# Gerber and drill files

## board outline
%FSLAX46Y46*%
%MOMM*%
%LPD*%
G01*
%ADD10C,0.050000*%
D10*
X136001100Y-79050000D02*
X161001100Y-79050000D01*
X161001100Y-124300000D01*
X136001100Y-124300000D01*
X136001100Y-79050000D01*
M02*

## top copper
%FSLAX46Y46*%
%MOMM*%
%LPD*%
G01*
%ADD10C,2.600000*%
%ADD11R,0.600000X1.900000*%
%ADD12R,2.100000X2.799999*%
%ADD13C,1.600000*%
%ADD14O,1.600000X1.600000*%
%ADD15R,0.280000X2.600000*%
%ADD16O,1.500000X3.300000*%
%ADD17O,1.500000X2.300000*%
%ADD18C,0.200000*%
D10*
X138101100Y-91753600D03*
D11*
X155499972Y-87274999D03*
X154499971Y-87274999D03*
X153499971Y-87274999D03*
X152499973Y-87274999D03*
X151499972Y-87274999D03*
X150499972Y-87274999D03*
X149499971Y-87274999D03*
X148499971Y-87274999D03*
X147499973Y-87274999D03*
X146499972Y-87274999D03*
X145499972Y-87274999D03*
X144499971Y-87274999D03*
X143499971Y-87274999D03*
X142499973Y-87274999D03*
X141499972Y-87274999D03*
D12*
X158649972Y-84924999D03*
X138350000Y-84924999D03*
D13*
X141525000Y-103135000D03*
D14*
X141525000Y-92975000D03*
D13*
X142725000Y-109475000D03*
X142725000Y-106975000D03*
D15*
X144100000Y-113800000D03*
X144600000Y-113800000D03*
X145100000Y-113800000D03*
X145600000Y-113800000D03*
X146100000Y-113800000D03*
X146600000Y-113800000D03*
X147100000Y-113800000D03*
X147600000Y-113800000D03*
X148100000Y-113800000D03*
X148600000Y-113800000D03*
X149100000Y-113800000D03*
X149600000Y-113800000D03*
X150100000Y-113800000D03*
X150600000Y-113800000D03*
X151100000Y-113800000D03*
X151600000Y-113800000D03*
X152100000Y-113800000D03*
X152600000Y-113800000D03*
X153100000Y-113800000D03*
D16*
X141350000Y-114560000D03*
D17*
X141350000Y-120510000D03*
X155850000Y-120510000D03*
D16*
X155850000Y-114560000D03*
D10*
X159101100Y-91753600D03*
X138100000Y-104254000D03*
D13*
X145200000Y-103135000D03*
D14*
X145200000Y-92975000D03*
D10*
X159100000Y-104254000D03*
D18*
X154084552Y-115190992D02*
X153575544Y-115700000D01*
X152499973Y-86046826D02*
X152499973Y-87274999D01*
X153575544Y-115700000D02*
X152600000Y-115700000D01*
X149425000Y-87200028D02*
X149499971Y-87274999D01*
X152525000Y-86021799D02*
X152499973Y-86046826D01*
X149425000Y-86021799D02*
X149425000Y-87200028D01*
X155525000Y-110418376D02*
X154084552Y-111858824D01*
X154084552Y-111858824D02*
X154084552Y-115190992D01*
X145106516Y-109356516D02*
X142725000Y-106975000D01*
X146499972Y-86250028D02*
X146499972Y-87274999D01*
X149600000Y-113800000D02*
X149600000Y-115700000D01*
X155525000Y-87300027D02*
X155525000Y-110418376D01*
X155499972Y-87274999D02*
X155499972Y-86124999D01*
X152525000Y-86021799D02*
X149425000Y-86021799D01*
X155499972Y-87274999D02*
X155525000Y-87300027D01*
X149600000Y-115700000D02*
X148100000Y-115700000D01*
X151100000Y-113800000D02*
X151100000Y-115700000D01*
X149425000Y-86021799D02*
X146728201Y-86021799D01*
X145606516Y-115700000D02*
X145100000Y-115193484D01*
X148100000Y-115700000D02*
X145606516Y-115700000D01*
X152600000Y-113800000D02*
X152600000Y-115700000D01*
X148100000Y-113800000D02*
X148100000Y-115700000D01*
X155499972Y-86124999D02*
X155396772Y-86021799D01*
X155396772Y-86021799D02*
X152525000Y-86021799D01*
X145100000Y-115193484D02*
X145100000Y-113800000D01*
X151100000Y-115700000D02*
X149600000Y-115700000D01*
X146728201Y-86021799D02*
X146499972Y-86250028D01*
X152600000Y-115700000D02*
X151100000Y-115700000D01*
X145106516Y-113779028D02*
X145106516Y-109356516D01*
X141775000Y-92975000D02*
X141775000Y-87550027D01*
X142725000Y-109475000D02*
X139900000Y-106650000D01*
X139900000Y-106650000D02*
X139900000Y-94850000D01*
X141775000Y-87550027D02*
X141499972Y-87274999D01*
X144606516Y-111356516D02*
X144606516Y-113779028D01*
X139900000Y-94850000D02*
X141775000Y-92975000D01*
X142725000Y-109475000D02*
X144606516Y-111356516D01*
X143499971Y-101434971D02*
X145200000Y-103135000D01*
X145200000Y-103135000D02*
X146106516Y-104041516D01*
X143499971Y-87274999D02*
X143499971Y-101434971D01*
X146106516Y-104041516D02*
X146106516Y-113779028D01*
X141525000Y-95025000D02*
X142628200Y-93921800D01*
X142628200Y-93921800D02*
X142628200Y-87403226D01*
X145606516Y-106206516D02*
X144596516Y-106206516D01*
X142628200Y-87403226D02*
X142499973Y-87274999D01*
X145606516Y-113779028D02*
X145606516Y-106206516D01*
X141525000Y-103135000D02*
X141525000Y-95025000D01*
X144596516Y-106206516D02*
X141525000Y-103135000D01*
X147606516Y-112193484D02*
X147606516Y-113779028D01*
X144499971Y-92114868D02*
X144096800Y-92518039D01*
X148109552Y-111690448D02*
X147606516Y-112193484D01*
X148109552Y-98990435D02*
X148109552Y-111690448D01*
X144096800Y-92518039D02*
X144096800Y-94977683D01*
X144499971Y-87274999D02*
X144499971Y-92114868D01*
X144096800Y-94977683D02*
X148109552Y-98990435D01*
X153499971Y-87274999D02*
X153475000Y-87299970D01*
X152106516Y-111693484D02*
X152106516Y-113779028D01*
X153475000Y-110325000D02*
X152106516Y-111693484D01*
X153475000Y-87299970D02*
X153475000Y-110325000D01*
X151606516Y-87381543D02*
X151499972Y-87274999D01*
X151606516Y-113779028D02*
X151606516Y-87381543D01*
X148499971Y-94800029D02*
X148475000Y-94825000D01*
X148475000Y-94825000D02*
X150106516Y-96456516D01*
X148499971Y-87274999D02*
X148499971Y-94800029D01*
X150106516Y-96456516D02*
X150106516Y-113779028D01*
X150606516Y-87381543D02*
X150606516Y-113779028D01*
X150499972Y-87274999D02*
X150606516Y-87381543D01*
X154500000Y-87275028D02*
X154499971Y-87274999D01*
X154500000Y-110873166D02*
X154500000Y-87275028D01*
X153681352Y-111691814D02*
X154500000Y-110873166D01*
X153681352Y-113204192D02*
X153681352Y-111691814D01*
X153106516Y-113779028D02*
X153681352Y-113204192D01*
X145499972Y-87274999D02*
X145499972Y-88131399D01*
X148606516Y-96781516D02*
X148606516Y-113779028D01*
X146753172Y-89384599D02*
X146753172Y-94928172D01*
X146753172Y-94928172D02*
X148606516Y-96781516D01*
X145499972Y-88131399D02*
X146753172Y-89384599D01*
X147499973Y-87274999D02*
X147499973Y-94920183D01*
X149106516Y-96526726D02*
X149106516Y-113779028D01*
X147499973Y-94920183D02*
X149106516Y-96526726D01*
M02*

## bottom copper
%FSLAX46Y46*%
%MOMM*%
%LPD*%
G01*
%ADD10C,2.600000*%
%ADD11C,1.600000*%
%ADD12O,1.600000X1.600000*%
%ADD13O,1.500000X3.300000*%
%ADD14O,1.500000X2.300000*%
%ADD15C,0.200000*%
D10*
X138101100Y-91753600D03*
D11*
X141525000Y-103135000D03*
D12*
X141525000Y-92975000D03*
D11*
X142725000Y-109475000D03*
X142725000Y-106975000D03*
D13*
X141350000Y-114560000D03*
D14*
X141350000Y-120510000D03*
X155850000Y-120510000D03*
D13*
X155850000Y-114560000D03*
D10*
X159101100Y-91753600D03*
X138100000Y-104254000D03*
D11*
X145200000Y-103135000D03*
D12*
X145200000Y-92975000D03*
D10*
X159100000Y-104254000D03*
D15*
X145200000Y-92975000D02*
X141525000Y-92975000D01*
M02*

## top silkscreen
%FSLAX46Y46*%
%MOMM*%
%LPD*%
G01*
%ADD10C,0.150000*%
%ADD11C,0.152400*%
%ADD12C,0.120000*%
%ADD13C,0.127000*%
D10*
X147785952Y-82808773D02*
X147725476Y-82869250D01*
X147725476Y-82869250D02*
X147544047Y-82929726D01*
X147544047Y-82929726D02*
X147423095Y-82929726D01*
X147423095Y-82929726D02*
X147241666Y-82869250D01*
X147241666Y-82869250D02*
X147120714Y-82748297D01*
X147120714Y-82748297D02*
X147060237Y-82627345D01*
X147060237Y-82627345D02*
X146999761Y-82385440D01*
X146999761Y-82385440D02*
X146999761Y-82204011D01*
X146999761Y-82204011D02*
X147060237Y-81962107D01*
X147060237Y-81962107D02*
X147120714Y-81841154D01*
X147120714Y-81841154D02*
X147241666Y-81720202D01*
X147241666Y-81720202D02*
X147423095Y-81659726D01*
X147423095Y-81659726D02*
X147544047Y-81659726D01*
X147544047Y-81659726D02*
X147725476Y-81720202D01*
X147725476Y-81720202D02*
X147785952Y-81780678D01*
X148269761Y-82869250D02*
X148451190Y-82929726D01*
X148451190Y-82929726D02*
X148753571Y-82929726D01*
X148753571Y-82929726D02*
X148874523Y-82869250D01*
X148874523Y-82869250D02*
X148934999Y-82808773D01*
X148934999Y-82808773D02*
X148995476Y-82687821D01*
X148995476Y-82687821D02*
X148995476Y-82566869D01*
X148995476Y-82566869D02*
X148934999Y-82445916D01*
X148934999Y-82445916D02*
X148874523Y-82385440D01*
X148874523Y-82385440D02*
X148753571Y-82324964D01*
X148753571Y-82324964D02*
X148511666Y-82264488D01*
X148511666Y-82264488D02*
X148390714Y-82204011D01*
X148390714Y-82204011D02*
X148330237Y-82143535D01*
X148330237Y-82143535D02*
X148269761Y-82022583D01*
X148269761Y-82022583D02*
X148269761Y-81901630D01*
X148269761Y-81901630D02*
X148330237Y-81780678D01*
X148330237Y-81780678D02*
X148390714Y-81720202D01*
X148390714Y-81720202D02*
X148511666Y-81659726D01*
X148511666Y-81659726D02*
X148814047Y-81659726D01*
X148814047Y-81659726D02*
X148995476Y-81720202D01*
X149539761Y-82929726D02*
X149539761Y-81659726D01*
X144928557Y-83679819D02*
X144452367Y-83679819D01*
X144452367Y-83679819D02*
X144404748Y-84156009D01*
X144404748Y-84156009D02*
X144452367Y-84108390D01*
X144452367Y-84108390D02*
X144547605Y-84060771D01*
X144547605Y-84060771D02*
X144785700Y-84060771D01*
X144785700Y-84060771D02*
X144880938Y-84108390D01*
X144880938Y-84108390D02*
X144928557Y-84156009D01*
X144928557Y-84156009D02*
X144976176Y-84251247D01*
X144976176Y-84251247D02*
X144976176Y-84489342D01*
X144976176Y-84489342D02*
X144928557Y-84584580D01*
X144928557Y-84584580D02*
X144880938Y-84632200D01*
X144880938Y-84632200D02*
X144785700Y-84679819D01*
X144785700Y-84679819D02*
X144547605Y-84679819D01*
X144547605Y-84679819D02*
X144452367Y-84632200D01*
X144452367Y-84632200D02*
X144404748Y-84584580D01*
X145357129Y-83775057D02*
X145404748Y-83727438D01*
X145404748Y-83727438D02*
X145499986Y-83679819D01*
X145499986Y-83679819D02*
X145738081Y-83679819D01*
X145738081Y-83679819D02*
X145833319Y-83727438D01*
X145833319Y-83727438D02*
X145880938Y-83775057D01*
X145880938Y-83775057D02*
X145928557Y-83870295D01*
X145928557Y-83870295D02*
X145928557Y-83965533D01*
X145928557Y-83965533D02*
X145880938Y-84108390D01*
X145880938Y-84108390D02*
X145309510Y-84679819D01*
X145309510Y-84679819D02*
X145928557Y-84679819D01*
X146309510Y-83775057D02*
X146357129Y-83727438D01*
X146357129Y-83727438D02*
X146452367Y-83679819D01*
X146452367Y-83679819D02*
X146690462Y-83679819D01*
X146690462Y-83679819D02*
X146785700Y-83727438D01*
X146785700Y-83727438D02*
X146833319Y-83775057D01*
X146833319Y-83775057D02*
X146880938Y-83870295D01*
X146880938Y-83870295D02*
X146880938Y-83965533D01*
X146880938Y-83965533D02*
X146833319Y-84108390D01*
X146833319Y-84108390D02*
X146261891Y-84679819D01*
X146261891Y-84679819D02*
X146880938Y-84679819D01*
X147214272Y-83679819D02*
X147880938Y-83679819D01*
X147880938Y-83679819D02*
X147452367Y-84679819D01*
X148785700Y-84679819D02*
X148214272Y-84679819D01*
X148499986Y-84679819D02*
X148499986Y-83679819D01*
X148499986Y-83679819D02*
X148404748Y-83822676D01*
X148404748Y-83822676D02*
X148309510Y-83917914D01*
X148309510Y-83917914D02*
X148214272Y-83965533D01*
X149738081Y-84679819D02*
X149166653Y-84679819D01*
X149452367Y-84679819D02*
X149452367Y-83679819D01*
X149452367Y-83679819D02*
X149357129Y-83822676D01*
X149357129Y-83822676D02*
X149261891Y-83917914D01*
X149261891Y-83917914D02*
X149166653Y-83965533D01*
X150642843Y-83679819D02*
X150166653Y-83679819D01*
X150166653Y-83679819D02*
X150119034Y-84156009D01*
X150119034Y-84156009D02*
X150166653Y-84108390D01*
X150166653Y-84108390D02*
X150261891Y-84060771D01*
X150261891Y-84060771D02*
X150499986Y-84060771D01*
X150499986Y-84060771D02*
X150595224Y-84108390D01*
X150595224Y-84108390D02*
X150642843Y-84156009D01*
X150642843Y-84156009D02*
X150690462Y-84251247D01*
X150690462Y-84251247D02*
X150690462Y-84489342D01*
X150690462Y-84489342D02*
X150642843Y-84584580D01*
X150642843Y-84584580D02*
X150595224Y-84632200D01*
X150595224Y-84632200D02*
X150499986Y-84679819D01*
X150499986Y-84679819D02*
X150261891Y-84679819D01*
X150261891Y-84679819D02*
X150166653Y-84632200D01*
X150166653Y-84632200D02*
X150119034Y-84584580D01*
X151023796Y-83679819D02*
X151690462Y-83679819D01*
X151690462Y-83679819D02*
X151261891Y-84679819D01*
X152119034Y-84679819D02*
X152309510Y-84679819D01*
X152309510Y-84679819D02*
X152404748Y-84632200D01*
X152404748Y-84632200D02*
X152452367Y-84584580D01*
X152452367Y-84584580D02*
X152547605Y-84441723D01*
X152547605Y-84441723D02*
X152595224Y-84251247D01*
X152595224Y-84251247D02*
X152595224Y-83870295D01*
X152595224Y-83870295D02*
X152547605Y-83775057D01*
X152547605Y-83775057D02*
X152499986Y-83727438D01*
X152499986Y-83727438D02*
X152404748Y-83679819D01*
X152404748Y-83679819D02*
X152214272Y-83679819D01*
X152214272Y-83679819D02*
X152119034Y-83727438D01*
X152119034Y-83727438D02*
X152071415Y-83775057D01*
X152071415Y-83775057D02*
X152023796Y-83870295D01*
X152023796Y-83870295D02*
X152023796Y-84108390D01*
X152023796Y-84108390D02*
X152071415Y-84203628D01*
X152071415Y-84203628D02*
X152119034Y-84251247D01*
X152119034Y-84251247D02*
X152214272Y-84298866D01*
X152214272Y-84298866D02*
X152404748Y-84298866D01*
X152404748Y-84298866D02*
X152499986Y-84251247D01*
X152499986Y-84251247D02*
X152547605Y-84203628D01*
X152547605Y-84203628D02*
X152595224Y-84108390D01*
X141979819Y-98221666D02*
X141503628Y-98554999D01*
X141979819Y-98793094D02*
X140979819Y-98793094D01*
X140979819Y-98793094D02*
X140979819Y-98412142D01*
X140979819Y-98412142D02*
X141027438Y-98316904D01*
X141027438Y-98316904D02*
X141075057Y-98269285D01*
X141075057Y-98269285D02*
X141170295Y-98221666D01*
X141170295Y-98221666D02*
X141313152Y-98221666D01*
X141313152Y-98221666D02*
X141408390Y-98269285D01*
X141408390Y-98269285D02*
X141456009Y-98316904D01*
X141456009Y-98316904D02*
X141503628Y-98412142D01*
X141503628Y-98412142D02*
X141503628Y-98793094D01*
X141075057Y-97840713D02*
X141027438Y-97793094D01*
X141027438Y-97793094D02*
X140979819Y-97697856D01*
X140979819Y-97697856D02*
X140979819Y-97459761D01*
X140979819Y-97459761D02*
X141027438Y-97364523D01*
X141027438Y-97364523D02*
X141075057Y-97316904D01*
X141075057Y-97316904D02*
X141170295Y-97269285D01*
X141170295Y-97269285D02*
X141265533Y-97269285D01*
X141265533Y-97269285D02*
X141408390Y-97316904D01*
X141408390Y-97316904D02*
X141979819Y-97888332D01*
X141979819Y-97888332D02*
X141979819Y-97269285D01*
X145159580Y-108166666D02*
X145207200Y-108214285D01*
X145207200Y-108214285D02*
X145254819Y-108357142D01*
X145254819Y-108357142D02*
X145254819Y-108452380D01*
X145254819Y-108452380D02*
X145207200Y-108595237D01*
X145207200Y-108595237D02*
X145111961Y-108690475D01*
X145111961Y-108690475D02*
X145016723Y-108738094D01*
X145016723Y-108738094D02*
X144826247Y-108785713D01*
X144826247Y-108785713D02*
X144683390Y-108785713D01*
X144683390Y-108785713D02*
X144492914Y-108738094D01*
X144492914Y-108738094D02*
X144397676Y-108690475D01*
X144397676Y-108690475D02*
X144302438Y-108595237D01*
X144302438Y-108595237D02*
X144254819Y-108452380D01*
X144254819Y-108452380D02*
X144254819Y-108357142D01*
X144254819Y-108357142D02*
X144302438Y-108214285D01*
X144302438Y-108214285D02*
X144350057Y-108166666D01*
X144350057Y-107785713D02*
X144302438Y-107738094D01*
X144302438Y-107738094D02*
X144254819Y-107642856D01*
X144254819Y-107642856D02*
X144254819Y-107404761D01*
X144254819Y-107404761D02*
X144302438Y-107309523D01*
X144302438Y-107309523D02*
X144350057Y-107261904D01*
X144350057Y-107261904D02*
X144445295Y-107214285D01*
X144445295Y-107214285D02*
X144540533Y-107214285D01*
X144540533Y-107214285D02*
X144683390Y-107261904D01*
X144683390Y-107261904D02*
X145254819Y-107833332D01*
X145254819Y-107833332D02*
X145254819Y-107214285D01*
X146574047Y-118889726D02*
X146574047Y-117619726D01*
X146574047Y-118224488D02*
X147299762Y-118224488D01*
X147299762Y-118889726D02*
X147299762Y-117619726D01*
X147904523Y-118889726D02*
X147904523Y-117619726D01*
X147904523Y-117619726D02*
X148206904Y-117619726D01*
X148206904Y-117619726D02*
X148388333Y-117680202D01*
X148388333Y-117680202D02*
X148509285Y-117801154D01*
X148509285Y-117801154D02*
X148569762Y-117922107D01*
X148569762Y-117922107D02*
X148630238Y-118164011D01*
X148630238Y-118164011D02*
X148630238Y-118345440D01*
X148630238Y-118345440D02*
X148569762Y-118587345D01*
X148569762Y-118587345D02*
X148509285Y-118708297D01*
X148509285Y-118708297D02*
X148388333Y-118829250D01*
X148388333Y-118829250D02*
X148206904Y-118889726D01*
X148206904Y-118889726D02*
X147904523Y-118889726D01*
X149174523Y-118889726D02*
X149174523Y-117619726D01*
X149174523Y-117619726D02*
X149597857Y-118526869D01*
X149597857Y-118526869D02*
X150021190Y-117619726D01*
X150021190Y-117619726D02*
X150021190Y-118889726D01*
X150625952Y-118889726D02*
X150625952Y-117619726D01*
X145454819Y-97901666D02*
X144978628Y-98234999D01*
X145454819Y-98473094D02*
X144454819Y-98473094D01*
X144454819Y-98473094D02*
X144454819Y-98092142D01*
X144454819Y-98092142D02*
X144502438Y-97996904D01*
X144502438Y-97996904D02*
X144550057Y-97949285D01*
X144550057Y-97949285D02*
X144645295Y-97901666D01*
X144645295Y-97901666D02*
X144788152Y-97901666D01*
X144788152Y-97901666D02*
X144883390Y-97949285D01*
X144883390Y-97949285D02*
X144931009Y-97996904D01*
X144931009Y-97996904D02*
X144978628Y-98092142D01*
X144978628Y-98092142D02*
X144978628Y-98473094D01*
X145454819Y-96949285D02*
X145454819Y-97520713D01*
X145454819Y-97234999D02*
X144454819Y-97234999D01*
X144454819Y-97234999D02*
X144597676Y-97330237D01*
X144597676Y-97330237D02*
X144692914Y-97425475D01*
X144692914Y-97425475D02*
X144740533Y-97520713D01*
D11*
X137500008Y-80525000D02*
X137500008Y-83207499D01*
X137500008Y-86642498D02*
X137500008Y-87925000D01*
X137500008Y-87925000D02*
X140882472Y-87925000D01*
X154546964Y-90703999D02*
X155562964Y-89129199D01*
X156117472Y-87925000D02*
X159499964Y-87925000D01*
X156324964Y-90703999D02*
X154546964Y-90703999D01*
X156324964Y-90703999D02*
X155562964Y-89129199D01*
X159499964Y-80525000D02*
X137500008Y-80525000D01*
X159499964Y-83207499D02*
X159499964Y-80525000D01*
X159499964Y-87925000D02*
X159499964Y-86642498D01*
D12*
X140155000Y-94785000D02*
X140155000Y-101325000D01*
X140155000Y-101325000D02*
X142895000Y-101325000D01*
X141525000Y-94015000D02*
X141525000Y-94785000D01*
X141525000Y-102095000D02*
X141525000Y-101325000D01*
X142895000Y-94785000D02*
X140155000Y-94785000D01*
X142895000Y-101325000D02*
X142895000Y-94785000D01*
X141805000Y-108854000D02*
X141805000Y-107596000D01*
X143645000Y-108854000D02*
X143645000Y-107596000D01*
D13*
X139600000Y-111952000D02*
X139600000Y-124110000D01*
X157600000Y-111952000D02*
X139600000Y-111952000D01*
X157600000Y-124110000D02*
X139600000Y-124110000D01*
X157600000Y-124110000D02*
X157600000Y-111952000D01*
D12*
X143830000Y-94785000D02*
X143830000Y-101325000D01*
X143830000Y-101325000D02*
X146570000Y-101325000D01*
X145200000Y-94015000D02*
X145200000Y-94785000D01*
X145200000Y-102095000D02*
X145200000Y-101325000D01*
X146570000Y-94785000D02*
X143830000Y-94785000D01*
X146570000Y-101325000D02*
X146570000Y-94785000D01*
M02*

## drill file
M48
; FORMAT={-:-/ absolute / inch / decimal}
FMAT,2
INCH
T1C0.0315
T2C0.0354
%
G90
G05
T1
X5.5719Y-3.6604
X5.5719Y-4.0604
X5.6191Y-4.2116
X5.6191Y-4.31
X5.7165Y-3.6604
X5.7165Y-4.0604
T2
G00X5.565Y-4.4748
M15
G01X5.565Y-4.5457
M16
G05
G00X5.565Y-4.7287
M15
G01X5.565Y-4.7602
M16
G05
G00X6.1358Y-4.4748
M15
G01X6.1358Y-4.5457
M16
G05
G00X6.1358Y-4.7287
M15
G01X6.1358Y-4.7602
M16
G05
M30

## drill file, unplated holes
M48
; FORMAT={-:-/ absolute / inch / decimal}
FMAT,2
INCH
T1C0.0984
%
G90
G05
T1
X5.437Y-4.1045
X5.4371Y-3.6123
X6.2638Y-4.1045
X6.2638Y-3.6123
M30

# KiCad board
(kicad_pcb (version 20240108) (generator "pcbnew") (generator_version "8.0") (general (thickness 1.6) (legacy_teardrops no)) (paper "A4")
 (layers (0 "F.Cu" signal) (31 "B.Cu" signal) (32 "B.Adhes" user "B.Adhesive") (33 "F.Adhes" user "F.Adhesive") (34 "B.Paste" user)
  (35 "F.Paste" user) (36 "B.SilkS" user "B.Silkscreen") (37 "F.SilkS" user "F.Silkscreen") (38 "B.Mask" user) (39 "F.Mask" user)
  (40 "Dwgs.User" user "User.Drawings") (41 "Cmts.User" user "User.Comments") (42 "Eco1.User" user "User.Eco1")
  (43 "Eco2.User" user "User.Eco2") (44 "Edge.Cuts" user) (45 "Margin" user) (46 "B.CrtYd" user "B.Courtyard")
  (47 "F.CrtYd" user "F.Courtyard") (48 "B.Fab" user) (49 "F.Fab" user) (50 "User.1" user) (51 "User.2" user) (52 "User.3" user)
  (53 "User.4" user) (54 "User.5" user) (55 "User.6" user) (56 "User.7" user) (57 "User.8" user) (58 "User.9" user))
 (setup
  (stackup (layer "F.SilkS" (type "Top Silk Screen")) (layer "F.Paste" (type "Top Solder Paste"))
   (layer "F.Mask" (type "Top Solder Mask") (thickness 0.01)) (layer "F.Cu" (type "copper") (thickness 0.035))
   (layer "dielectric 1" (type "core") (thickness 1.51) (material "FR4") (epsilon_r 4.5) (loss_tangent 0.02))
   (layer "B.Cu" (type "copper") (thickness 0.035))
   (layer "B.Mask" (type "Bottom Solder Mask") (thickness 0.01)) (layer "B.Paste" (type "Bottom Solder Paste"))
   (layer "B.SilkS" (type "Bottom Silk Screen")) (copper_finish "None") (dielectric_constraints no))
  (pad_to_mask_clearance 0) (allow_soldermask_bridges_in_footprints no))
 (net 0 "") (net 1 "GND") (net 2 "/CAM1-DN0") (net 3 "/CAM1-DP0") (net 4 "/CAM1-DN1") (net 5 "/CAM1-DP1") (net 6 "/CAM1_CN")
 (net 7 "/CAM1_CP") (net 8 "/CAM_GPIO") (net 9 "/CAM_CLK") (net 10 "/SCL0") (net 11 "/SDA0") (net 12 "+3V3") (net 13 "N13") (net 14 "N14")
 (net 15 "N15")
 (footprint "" (layer "F.Cu") (at 138.1011 91.7536)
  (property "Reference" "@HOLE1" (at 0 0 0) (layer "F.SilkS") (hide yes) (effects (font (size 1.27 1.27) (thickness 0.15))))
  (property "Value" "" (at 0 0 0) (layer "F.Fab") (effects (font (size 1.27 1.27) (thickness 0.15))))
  (pad "" np_thru_hole circle (at 0 0) (size 2.6 2.6) (drill 2.5) (layers "F&B.Cu" "*.Mask")))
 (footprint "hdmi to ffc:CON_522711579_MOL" (layer "F.Cu") (at 148.499986 84.225 180)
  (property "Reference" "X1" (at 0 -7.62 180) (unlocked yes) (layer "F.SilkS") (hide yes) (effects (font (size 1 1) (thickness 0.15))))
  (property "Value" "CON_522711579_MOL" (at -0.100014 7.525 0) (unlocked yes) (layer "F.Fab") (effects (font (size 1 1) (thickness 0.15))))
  (fp_line (start 10.999978 3.7) (end 10.999978 1.017501) (stroke (width 0.1524) (type solid)) (layer "F.SilkS"))
  (fp_line (start 10.999978 -2.417498) (end 10.999978 -3.7) (stroke (width 0.1524) (type solid)) (layer "F.SilkS"))
  (fp_line (start 10.999978 -3.7) (end 7.617514 -3.7) (stroke (width 0.1524) (type solid)) (layer "F.SilkS"))
  (fp_line (start -6.046978 -6.478999) (end -7.062978 -4.904199) (stroke (width 0.1524) (type solid)) (layer "F.SilkS"))
  (fp_line (start -7.617486 -3.7) (end -10.999978 -3.7) (stroke (width 0.1524) (type solid)) (layer "F.SilkS"))
  (fp_line (start -7.824978 -6.478999) (end -6.046978 -6.478999) (stroke (width 0.1524) (type solid)) (layer "F.SilkS"))
  (fp_line (start -7.824978 -6.478999) (end -7.062978 -4.904199) (stroke (width 0.1524) (type solid)) (layer "F.SilkS"))
  (fp_line (start -10.999978 3.7) (end 10.999978 3.7) (stroke (width 0.1524) (type solid)) (layer "F.SilkS"))
  (fp_line (start -10.999978 1.017501) (end -10.999978 3.7) (stroke (width 0.1524) (type solid)) (layer "F.SilkS"))
  (fp_line (start -10.999978 -3.7) (end -10.999978 -2.417498) (stroke (width 0.1524) (type solid)) (layer "F.SilkS"))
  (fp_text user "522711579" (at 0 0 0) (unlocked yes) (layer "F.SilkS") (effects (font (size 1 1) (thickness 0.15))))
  (pad "1" smd rect (at -6.999986 -3.049999 180) (size 0.6 1.9) (layers "F.Cu" "F.Paste" "F.Mask") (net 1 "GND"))
  (pad "2" smd rect (at -5.999985 -3.049999 180) (size 0.6 1.9) (layers "F.Cu" "F.Paste" "F.Mask") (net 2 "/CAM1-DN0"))
  (pad "3" smd rect (at -4.999985 -3.049999 180) (size 0.6 1.9) (layers "F.Cu" "F.Paste" "F.Mask") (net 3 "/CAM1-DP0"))
  (pad "4" smd rect (at -3.999987 -3.049999 180) (size 0.6 1.9) (layers "F.Cu" "F.Paste" "F.Mask") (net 1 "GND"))
  (pad "5" smd rect (at -2.999986 -3.049999 180) (size 0.6 1.9) (layers "F.Cu" "F.Paste" "F.Mask") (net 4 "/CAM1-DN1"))
  (pad "6" smd rect (at -1.999986 -3.049999 180) (size 0.6 1.9) (layers "F.Cu" "F.Paste" "F.Mask") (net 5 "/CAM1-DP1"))
  (pad "7" smd rect (at -0.999985 -3.049999 180) (size 0.6 1.9) (layers "F.Cu" "F.Paste" "F.Mask") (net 1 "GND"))
  (pad "8" smd rect (at 0.000015 -3.049999 180) (size 0.6 1.9) (layers "F.Cu" "F.Paste" "F.Mask") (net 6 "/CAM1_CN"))
  (pad "9" smd rect (at 1.000013 -3.049999 180) (size 0.6 1.9) (layers "F.Cu" "F.Paste" "F.Mask") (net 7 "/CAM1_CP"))
  (pad "10" smd rect (at 2.000014 -3.049999 180) (size 0.6 1.9) (layers "F.Cu" "F.Paste" "F.Mask") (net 1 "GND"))
  (pad "11" smd rect (at 3.000014 -3.049999 180) (size 0.6 1.9) (layers "F.Cu" "F.Paste" "F.Mask") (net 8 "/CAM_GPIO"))
  (pad "12" smd rect (at 4.000015 -3.049999 180) (size 0.6 1.9) (layers "F.Cu" "F.Paste" "F.Mask") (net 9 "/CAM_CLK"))
  (pad "13" smd rect (at 5.000015 -3.049999 180) (size 0.6 1.9) (layers "F.Cu" "F.Paste" "F.Mask") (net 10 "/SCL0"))
  (pad "14" smd rect (at 6.000013 -3.049999 180) (size 0.6 1.9) (layers "F.Cu" "F.Paste" "F.Mask") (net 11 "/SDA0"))
  (pad "15" smd rect (at 7.000014 -3.049999 180) (size 0.6 1.9) (layers "F.Cu" "F.Paste" "F.Mask") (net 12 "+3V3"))
  (pad "P1" smd rect (at -10.149986 -0.699999 180) (size 2.1 2.799999) (layers "F.Cu" "F.Paste" "F.Mask"))
  (pad "P2" smd rect (at 10.149986 -0.699999 180) (size 2.1 2.799999) (layers "F.Cu" "F.Paste" "F.Mask")))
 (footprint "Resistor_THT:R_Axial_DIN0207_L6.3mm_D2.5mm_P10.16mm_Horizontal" (layer "F.Cu") (at 141.525 103.135 90)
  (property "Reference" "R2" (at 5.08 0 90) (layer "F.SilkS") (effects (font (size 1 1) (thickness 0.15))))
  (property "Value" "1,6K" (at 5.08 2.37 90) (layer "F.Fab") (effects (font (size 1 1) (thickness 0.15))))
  (fp_line (start 8.35 -1.37) (end 1.81 -1.37) (stroke (width 0.12) (type solid)) (layer "F.SilkS"))
  (fp_line (start 1.81 -1.37) (end 1.81 1.37) (stroke (width 0.12) (type solid)) (layer "F.SilkS"))
  (fp_line (start 9.12 0) (end 8.35 0) (stroke (width 0.12) (type solid)) (layer "F.SilkS"))
  (fp_line (start 1.04 0) (end 1.81 0) (stroke (width 0.12) (type solid)) (layer "F.SilkS"))
  (fp_line (start 8.35 1.37) (end 8.35 -1.37) (stroke (width 0.12) (type solid)) (layer "F.SilkS"))
  (fp_line (start 1.81 1.37) (end 8.35 1.37) (stroke (width 0.12) (type solid)) (layer "F.SilkS"))
  (pad "1" thru_hole circle (at 0 0 90) (size 1.6 1.6) (drill 0.8) (layers "*.Cu" "*.Mask") (remove_unused_layers no) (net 11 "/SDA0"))
  (pad "2" thru_hole oval (at 10.16 0 90) (size 1.6 1.6) (drill 0.8) (layers "*.Cu" "*.Mask") (remove_unused_layers no) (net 12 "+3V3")))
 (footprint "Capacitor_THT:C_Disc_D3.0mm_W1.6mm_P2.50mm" (layer "F.Cu") (at 142.725 109.475 90)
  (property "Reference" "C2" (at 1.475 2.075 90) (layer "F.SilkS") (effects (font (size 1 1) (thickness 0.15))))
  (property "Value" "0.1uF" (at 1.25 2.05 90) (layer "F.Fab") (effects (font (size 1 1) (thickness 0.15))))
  (fp_line (start 0.621 -0.92) (end 1.879 -0.92) (stroke (width 0.12) (type solid)) (layer "F.SilkS"))
  (fp_line (start 0.621 0.92) (end 1.879 0.92) (stroke (width 0.12) (type solid)) (layer "F.SilkS"))
  (pad "1" thru_hole circle (at 0 0 90) (size 1.6 1.6) (drill 0.8) (layers "*.Cu" "*.Mask") (remove_unused_layers no) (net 12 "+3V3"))
  (pad "2" thru_hole circle (at 2.5 0 90) (size 1.6 1.6) (drill 0.8) (layers "*.Cu" "*.Mask") (remove_unused_layers no) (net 1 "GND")))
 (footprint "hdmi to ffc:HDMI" (layer "F.Cu") (at 148.6 115.01)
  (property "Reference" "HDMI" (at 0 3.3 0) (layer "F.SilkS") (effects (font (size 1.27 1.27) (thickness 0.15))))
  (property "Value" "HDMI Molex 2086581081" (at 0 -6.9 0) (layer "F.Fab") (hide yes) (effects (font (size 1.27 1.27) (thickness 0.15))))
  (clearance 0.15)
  (fp_line (start -9 -3.058) (end -9 9.1) (stroke (width 0.127) (type solid)) (layer "F.SilkS"))
  (fp_line (start 9 -3.058) (end -9 -3.058) (stroke (width 0.127) (type solid)) (layer "F.SilkS"))
  (fp_line (start 9 9.1) (end -9 9.1) (stroke (width 0.127) (type solid)) (layer "F.SilkS"))
  (fp_line (start 9 9.1) (end 9 -3.058) (stroke (width 0.127) (type solid)) (layer "F.SilkS"))
  (pad "P$1" smd rect (at -4.5 -1.21 90) (size 2.6 0.28) (layers "F.Cu" "F.Paste" "F.Mask") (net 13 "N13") (clearance 0.1)
   (thermal_bridge_angle 0))
  (pad "P$2" smd rect (at -4 -1.21 90) (size 2.6 0.28) (layers "F.Cu" "F.Paste" "F.Mask") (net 12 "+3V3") (clearance 0.1)
   (thermal_bridge_angle 0))
  (pad "P$3" smd rect (at -3.5 -1.21 90) (size 2.6 0.28) (layers "F.Cu" "F.Paste" "F.Mask") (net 1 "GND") (clearance 0.1)
   (thermal_bridge_angle 0))
  (pad "P$4" smd rect (at -3 -1.21 90) (size 2.6 0.28) (layers "F.Cu" "F.Paste" "F.Mask") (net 11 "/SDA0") (clearance 0.1)
   (thermal_bridge_angle 0))
  (pad "P$5" smd rect (at -2.5 -1.21 90) (size 2.6 0.28) (layers "F.Cu" "F.Paste" "F.Mask") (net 10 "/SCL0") (clearance 0.1)
   (thermal_bridge_angle 0))
  (pad "P$6" smd rect (at -2 -1.21 90) (size 2.6 0.28) (layers "F.Cu" "F.Paste" "F.Mask") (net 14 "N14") (clearance 0.1)
   (thermal_bridge_angle 0))
  (pad "P$7" smd rect (at -1.5 -1.21 90) (size 2.6 0.28) (layers "F.Cu" "F.Paste" "F.Mask") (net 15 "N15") (clearance 0.1)
   (thermal_bridge_angle 0))
  (pad "P$8" smd rect (at -1 -1.21 90) (size 2.6 0.28) (layers "F.Cu" "F.Paste" "F.Mask") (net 9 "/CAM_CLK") (clearance 0.1)
   (thermal_bridge_angle 0))
  (pad "P$9" smd rect (at -0.5 -1.21 90) (size 2.6 0.28) (layers "F.Cu" "F.Paste" "F.Mask") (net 1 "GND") (clearance 0.1)
   (thermal_bridge_angle 0))
  (pad "P$10" smd rect (at 0 -1.21 90) (size 2.6 0.28) (layers "F.Cu" "F.Paste" "F.Mask") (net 8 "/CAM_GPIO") (clearance 0.1)
   (thermal_bridge_angle 0))
  (pad "P$11" smd rect (at 0.5 -1.21 90) (size 2.6 0.28) (layers "F.Cu" "F.Paste" "F.Mask") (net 7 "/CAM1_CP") (clearance 0.1)
   (thermal_bridge_angle 0))
  (pad "P$12" smd rect (at 1 -1.21 90) (size 2.6 0.28) (layers "F.Cu" "F.Paste" "F.Mask") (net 1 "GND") (clearance 0.1)
   (thermal_bridge_angle 0))
  (pad "P$13" smd rect (at 1.5 -1.21 90) (size 2.6 0.28) (layers "F.Cu" "F.Paste" "F.Mask") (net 6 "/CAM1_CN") (clearance 0.1)
   (thermal_bridge_angle 0))
  (pad "P$14" smd rect (at 2 -1.21 90) (size 2.6 0.28) (layers "F.Cu" "F.Paste" "F.Mask") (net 5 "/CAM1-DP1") (clearance 0.1)
   (thermal_bridge_angle 0))
  (pad "P$15" smd rect (at 2.5 -1.21 90) (size 2.6 0.28) (layers "F.Cu" "F.Paste" "F.Mask") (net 1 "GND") (clearance 0.1)
   (thermal_bridge_angle 0))
  (pad "P$16" smd rect (at 3 -1.21 90) (size 2.6 0.28) (layers "F.Cu" "F.Paste" "F.Mask") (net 4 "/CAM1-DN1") (clearance 0.1)
   (thermal_bridge_angle 0))
  (pad "P$17" smd rect (at 3.5 -1.21 90) (size 2.6 0.28) (layers "F.Cu" "F.Paste" "F.Mask") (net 3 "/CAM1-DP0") (clearance 0.1)
   (thermal_bridge_angle 0))
  (pad "P$18" smd rect (at 4 -1.21 90) (size 2.6 0.28) (layers "F.Cu" "F.Paste" "F.Mask") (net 1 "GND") (clearance 0.1)
   (thermal_bridge_angle 0))
  (pad "P$19" smd rect (at 4.5 -1.21 90) (size 2.6 0.28) (layers "F.Cu" "F.Paste" "F.Mask") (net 2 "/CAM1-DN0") (clearance 0.1)
   (thermal_bridge_angle 0))
  (pad "P$20" thru_hole oval (at -7.25 -0.45) (size 1.5 3.3) (drill oval 0.9 2.7) (layers "*.Cu" "*.Mask") (remove_unused_layers no)
   (solder_mask_margin 0.1016) (thermal_bridge_angle 0))
  (pad "P$21" thru_hole oval (at -7.25 5.5) (size 1.5 2.3) (drill oval 0.9 1.7) (layers "*.Cu" "*.Mask") (remove_unused_layers no)
   (solder_mask_margin 0.1016) (thermal_bridge_angle 0))
  (pad "P$22" thru_hole oval (at 7.25 5.5) (size 1.5 2.3) (drill oval 0.9 1.7) (layers "*.Cu" "*.Mask") (remove_unused_layers no)
   (solder_mask_margin 0.1016) (thermal_bridge_angle 0))
  (pad "P$23" thru_hole oval (at 7.25 -0.45) (size 1.5 3.3) (drill oval 0.9 2.7) (layers "*.Cu" "*.Mask") (remove_unused_layers no)
   (solder_mask_margin 0.1016) (thermal_bridge_angle 0)))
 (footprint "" (layer "F.Cu") (at 159.1011 91.7536)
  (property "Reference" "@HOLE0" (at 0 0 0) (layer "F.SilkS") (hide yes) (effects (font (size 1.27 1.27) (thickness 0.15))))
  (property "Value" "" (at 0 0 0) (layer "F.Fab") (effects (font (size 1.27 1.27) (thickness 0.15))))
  (pad "" np_thru_hole circle (at 0 0) (size 2.6 2.6) (drill 2.5) (layers "F&B.Cu" "*.Mask")))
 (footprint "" (layer "F.Cu") (at 138.1 104.254)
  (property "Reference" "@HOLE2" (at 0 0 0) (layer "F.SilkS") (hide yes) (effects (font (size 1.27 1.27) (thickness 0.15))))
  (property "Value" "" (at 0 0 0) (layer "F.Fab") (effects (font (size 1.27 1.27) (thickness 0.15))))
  (pad "" np_thru_hole circle (at 0 0) (size 2.6 2.6) (drill 2.5) (layers "F&B.Cu" "*.Mask")))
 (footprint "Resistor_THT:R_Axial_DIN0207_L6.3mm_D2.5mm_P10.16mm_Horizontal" (layer "F.Cu") (at 145.2 103.135 90)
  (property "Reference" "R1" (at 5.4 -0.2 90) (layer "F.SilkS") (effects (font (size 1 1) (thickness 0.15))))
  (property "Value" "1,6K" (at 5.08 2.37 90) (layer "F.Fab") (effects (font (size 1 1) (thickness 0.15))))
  (fp_line (start 8.35 -1.37) (end 1.81 -1.37) (stroke (width 0.12) (type solid)) (layer "F.SilkS"))
  (fp_line (start 1.81 -1.37) (end 1.81 1.37) (stroke (width 0.12) (type solid)) (layer "F.SilkS"))
  (fp_line (start 9.12 0) (end 8.35 0) (stroke (width 0.12) (type solid)) (layer "F.SilkS"))
  (fp_line (start 1.04 0) (end 1.81 0) (stroke (width 0.12) (type solid)) (layer "F.SilkS"))
  (fp_line (start 8.35 1.37) (end 8.35 -1.37) (stroke (width 0.12) (type solid)) (layer "F.SilkS"))
  (fp_line (start 1.81 1.37) (end 8.35 1.37) (stroke (width 0.12) (type solid)) (layer "F.SilkS"))
  (pad "1" thru_hole circle (at 0 0 90) (size 1.6 1.6) (drill 0.8) (layers "*.Cu" "*.Mask") (remove_unused_layers no) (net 10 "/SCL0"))
  (pad "2" thru_hole oval (at 10.16 0 90) (size 1.6 1.6) (drill 0.8) (layers "*.Cu" "*.Mask") (remove_unused_layers no) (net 12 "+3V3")))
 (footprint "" (layer "F.Cu") (at 159.1 104.254)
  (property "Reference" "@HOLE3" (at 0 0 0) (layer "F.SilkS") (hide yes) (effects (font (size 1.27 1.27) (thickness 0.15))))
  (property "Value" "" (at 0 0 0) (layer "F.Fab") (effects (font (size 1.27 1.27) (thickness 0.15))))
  (pad "" np_thru_hole circle (at 0 0) (size 2.6 2.6) (drill 2.5) (layers "F&B.Cu" "*.Mask")))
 (gr_rect (start 136.0011 79.05) (end 161.0011 124.3) (stroke (width 0.05) (type default)) (fill none) (layer "Edge.Cuts"))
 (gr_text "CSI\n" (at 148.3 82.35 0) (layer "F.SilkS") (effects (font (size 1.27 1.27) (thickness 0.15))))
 (segment (start 154.084552 115.190992) (end 153.575544 115.7) (width 0.2) (layer "F.Cu") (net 1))
 (segment (start 152.499973 86.046826) (end 152.499973 87.274999) (width 0.2) (layer "F.Cu") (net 1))
 (segment (start 153.575544 115.7) (end 152.6 115.7) (width 0.2) (layer "F.Cu") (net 1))
 (segment (start 149.425 87.200028) (end 149.499971 87.274999) (width 0.2) (layer "F.Cu") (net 1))
 (segment (start 152.525 86.021799) (end 152.499973 86.046826) (width 0.2) (layer "F.Cu") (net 1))
 (segment (start 149.425 86.021799) (end 149.425 87.200028) (width 0.2) (layer "F.Cu") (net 1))
 (segment (start 155.525 110.418376) (end 154.084552 111.858824) (width 0.2) (layer "F.Cu") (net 1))
 (segment (start 154.084552 111.858824) (end 154.084552 115.190992) (width 0.2) (layer "F.Cu") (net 1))
 (segment (start 145.106516 109.356516) (end 142.725 106.975) (width 0.2) (layer "F.Cu") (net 1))
 (segment (start 146.499972 86.250028) (end 146.499972 87.274999) (width 0.2) (layer "F.Cu") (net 1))
 (segment (start 149.6 113.8) (end 149.6 115.7) (width 0.2) (layer "F.Cu") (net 1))
 (segment (start 155.525 87.300027) (end 155.525 110.418376) (width 0.2) (layer "F.Cu") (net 1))
 (segment (start 155.499972 87.274999) (end 155.499972 86.124999) (width 0.2) (layer "F.Cu") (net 1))
 (segment (start 152.525 86.021799) (end 149.425 86.021799) (width 0.2) (layer "F.Cu") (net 1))
 (segment (start 155.499972 87.274999) (end 155.525 87.300027) (width 0.2) (layer "F.Cu") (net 1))
 (segment (start 149.6 115.7) (end 148.1 115.7) (width 0.2) (layer "F.Cu") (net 1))
 (segment (start 151.1 113.8) (end 151.1 115.7) (width 0.2) (layer "F.Cu") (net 1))
 (segment (start 149.425 86.021799) (end 146.728201 86.021799) (width 0.2) (layer "F.Cu") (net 1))
 (segment (start 145.606516 115.7) (end 145.1 115.193484) (width 0.2) (layer "F.Cu") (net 1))
 (segment (start 148.1 115.7) (end 145.606516 115.7) (width 0.2) (layer "F.Cu") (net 1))
 (segment (start 152.6 113.8) (end 152.6 115.7) (width 0.2) (layer "F.Cu") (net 1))
 (segment (start 148.1 113.8) (end 148.1 115.7) (width 0.2) (layer "F.Cu") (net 1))
 (segment (start 155.499972 86.124999) (end 155.396772 86.021799) (width 0.2) (layer "F.Cu") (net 1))
 (segment (start 155.396772 86.021799) (end 152.525 86.021799) (width 0.2) (layer "F.Cu") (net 1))
 (segment (start 145.1 115.193484) (end 145.1 113.8) (width 0.2) (layer "F.Cu") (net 1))
 (segment (start 151.1 115.7) (end 149.6 115.7) (width 0.2) (layer "F.Cu") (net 1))
 (segment (start 146.728201 86.021799) (end 146.499972 86.250028) (width 0.2) (layer "F.Cu") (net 1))
 (segment (start 152.6 115.7) (end 151.1 115.7) (width 0.2) (layer "F.Cu") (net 1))
 (segment (start 145.106516 113.779028) (end 145.106516 109.356516) (width 0.2) (layer "F.Cu") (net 1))
 (segment (start 141.775 92.975) (end 141.775 87.550027) (width 0.2) (layer "F.Cu") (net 12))
 (segment (start 142.725 109.475) (end 139.9 106.65) (width 0.2) (layer "F.Cu") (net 12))
 (segment (start 139.9 106.65) (end 139.9 94.85) (width 0.2) (layer "F.Cu") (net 12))
 (segment (start 141.775 87.550027) (end 141.499972 87.274999) (width 0.2) (layer "F.Cu") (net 12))
 (segment (start 144.606516 111.356516) (end 144.606516 113.779028) (width 0.2) (layer "F.Cu") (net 12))
 (segment (start 139.9 94.85) (end 141.775 92.975) (width 0.2) (layer "F.Cu") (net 12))
 (segment (start 142.725 109.475) (end 144.606516 111.356516) (width 0.2) (layer "F.Cu") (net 12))
 (segment (start 145.2 92.975) (end 141.525 92.975) (width 0.2) (layer "B.Cu") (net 12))
 (segment (start 143.499971 101.434971) (end 145.2 103.135) (width 0.2) (layer "F.Cu") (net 10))
 (segment (start 145.2 103.135) (end 146.106516 104.041516) (width 0.2) (layer "F.Cu") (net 10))
 (segment (start 143.499971 87.274999) (end 143.499971 101.434971) (width 0.2) (layer "F.Cu") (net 10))
 (segment (start 146.106516 104.041516) (end 146.106516 113.779028) (width 0.2) (layer "F.Cu") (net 10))
 (segment (start 141.525 95.025) (end 142.6282 93.9218) (width 0.2) (layer "F.Cu") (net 11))
 (segment (start 142.6282 93.9218) (end 142.6282 87.403226) (width 0.2) (layer "F.Cu") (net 11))
 (segment (start 145.606516 106.206516) (end 144.596516 106.206516) (width 0.2) (layer "F.Cu") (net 11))
 (segment (start 142.6282 87.403226) (end 142.499973 87.274999) (width 0.2) (layer "F.Cu") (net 11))
 (segment (start 145.606516 113.779028) (end 145.606516 106.206516) (width 0.2) (layer "F.Cu") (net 11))
 (segment (start 141.525 103.135) (end 141.525 95.025) (width 0.2) (layer "F.Cu") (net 11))
 (segment (start 144.596516 106.206516) (end 141.525 103.135) (width 0.2) (layer "F.Cu") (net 11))
 (segment (start 147.606516 112.193484) (end 147.606516 113.779028) (width 0.2) (layer "F.Cu") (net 9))
 (segment (start 144.499971 92.114868) (end 144.0968 92.518039) (width 0.2) (layer "F.Cu") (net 9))
 (segment (start 148.109552 111.690448) (end 147.606516 112.193484) (width 0.2) (layer "F.Cu") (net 9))
 (segment (start 148.109552 98.990435) (end 148.109552 111.690448) (width 0.2) (layer "F.Cu") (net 9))
 (segment (start 144.0968 92.518039) (end 144.0968 94.977683) (width 0.2) (layer "F.Cu") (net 9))
 (segment (start 144.499971 87.274999) (end 144.499971 92.114868) (width 0.2) (layer "F.Cu") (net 9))
 (segment (start 144.0968 94.977683) (end 148.109552 98.990435) (width 0.2) (layer "F.Cu") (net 9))
 (segment (start 153.499971 87.274999) (end 153.475 87.29997) (width 0.2) (layer "F.Cu") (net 3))
 (segment (start 152.106516 111.693484) (end 152.106516 113.779028) (width 0.2) (layer "F.Cu") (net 3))
 (segment (start 153.475 110.325) (end 152.106516 111.693484) (width 0.2) (layer "F.Cu") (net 3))
 (segment (start 153.475 87.29997) (end 153.475 110.325) (width 0.2) (layer "F.Cu") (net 3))
 (segment (start 151.606516 87.381543) (end 151.499972 87.274999) (width 0.2) (layer "F.Cu") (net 4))
 (segment (start 151.606516 113.779028) (end 151.606516 87.381543) (width 0.2) (layer "F.Cu") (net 4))
 (segment (start 148.499971 94.800029) (end 148.475 94.825) (width 0.2) (layer "F.Cu") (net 6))
 (segment (start 148.475 94.825) (end 150.106516 96.456516) (width 0.2) (layer "F.Cu") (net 6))
 (segment (start 148.499971 87.274999) (end 148.499971 94.800029) (width 0.2) (layer "F.Cu") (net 6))
 (segment (start 150.106516 96.456516) (end 150.106516 113.779028) (width 0.2) (layer "F.Cu") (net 6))
 (segment (start 150.606516 87.381543) (end 150.606516 113.779028) (width 0.2) (layer "F.Cu") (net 5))
 (segment (start 150.499972 87.274999) (end 150.606516 87.381543) (width 0.2) (layer "F.Cu") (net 5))
 (segment (start 154.5 87.275028) (end 154.499971 87.274999) (width 0.2) (layer "F.Cu") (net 2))
 (segment (start 154.5 110.873166) (end 154.5 87.275028) (width 0.2) (layer "F.Cu") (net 2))
 (segment (start 153.681352 111.691814) (end 154.5 110.873166) (width 0.2) (layer "F.Cu") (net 2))
 (segment (start 153.681352 113.204192) (end 153.681352 111.691814) (width 0.2) (layer "F.Cu") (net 2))
 (segment (start 153.106516 113.779028) (end 153.681352 113.204192) (width 0.2) (layer "F.Cu") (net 2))
 (segment (start 145.499972 87.274999) (end 145.499972 88.131399) (width 0.2) (layer "F.Cu") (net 8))
 (segment (start 148.606516 96.781516) (end 148.606516 113.779028) (width 0.2) (layer "F.Cu") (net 8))
 (segment (start 146.753172 89.384599) (end 146.753172 94.928172) (width 0.2) (layer "F.Cu") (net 8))
 (segment (start 146.753172 94.928172) (end 148.606516 96.781516) (width 0.2) (layer "F.Cu") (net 8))
 (segment (start 145.499972 88.131399) (end 146.753172 89.384599) (width 0.2) (layer "F.Cu") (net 8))
 (segment (start 147.499973 87.274999) (end 147.499973 94.920183) (width 0.2) (layer "F.Cu") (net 7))
 (segment (start 149.106516 96.526726) (end 149.106516 113.779028) (width 0.2) (layer "F.Cu") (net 7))
 (segment (start 147.499973 94.920183) (end 149.106516 96.526726) (width 0.2) (layer "F.Cu") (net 7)))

